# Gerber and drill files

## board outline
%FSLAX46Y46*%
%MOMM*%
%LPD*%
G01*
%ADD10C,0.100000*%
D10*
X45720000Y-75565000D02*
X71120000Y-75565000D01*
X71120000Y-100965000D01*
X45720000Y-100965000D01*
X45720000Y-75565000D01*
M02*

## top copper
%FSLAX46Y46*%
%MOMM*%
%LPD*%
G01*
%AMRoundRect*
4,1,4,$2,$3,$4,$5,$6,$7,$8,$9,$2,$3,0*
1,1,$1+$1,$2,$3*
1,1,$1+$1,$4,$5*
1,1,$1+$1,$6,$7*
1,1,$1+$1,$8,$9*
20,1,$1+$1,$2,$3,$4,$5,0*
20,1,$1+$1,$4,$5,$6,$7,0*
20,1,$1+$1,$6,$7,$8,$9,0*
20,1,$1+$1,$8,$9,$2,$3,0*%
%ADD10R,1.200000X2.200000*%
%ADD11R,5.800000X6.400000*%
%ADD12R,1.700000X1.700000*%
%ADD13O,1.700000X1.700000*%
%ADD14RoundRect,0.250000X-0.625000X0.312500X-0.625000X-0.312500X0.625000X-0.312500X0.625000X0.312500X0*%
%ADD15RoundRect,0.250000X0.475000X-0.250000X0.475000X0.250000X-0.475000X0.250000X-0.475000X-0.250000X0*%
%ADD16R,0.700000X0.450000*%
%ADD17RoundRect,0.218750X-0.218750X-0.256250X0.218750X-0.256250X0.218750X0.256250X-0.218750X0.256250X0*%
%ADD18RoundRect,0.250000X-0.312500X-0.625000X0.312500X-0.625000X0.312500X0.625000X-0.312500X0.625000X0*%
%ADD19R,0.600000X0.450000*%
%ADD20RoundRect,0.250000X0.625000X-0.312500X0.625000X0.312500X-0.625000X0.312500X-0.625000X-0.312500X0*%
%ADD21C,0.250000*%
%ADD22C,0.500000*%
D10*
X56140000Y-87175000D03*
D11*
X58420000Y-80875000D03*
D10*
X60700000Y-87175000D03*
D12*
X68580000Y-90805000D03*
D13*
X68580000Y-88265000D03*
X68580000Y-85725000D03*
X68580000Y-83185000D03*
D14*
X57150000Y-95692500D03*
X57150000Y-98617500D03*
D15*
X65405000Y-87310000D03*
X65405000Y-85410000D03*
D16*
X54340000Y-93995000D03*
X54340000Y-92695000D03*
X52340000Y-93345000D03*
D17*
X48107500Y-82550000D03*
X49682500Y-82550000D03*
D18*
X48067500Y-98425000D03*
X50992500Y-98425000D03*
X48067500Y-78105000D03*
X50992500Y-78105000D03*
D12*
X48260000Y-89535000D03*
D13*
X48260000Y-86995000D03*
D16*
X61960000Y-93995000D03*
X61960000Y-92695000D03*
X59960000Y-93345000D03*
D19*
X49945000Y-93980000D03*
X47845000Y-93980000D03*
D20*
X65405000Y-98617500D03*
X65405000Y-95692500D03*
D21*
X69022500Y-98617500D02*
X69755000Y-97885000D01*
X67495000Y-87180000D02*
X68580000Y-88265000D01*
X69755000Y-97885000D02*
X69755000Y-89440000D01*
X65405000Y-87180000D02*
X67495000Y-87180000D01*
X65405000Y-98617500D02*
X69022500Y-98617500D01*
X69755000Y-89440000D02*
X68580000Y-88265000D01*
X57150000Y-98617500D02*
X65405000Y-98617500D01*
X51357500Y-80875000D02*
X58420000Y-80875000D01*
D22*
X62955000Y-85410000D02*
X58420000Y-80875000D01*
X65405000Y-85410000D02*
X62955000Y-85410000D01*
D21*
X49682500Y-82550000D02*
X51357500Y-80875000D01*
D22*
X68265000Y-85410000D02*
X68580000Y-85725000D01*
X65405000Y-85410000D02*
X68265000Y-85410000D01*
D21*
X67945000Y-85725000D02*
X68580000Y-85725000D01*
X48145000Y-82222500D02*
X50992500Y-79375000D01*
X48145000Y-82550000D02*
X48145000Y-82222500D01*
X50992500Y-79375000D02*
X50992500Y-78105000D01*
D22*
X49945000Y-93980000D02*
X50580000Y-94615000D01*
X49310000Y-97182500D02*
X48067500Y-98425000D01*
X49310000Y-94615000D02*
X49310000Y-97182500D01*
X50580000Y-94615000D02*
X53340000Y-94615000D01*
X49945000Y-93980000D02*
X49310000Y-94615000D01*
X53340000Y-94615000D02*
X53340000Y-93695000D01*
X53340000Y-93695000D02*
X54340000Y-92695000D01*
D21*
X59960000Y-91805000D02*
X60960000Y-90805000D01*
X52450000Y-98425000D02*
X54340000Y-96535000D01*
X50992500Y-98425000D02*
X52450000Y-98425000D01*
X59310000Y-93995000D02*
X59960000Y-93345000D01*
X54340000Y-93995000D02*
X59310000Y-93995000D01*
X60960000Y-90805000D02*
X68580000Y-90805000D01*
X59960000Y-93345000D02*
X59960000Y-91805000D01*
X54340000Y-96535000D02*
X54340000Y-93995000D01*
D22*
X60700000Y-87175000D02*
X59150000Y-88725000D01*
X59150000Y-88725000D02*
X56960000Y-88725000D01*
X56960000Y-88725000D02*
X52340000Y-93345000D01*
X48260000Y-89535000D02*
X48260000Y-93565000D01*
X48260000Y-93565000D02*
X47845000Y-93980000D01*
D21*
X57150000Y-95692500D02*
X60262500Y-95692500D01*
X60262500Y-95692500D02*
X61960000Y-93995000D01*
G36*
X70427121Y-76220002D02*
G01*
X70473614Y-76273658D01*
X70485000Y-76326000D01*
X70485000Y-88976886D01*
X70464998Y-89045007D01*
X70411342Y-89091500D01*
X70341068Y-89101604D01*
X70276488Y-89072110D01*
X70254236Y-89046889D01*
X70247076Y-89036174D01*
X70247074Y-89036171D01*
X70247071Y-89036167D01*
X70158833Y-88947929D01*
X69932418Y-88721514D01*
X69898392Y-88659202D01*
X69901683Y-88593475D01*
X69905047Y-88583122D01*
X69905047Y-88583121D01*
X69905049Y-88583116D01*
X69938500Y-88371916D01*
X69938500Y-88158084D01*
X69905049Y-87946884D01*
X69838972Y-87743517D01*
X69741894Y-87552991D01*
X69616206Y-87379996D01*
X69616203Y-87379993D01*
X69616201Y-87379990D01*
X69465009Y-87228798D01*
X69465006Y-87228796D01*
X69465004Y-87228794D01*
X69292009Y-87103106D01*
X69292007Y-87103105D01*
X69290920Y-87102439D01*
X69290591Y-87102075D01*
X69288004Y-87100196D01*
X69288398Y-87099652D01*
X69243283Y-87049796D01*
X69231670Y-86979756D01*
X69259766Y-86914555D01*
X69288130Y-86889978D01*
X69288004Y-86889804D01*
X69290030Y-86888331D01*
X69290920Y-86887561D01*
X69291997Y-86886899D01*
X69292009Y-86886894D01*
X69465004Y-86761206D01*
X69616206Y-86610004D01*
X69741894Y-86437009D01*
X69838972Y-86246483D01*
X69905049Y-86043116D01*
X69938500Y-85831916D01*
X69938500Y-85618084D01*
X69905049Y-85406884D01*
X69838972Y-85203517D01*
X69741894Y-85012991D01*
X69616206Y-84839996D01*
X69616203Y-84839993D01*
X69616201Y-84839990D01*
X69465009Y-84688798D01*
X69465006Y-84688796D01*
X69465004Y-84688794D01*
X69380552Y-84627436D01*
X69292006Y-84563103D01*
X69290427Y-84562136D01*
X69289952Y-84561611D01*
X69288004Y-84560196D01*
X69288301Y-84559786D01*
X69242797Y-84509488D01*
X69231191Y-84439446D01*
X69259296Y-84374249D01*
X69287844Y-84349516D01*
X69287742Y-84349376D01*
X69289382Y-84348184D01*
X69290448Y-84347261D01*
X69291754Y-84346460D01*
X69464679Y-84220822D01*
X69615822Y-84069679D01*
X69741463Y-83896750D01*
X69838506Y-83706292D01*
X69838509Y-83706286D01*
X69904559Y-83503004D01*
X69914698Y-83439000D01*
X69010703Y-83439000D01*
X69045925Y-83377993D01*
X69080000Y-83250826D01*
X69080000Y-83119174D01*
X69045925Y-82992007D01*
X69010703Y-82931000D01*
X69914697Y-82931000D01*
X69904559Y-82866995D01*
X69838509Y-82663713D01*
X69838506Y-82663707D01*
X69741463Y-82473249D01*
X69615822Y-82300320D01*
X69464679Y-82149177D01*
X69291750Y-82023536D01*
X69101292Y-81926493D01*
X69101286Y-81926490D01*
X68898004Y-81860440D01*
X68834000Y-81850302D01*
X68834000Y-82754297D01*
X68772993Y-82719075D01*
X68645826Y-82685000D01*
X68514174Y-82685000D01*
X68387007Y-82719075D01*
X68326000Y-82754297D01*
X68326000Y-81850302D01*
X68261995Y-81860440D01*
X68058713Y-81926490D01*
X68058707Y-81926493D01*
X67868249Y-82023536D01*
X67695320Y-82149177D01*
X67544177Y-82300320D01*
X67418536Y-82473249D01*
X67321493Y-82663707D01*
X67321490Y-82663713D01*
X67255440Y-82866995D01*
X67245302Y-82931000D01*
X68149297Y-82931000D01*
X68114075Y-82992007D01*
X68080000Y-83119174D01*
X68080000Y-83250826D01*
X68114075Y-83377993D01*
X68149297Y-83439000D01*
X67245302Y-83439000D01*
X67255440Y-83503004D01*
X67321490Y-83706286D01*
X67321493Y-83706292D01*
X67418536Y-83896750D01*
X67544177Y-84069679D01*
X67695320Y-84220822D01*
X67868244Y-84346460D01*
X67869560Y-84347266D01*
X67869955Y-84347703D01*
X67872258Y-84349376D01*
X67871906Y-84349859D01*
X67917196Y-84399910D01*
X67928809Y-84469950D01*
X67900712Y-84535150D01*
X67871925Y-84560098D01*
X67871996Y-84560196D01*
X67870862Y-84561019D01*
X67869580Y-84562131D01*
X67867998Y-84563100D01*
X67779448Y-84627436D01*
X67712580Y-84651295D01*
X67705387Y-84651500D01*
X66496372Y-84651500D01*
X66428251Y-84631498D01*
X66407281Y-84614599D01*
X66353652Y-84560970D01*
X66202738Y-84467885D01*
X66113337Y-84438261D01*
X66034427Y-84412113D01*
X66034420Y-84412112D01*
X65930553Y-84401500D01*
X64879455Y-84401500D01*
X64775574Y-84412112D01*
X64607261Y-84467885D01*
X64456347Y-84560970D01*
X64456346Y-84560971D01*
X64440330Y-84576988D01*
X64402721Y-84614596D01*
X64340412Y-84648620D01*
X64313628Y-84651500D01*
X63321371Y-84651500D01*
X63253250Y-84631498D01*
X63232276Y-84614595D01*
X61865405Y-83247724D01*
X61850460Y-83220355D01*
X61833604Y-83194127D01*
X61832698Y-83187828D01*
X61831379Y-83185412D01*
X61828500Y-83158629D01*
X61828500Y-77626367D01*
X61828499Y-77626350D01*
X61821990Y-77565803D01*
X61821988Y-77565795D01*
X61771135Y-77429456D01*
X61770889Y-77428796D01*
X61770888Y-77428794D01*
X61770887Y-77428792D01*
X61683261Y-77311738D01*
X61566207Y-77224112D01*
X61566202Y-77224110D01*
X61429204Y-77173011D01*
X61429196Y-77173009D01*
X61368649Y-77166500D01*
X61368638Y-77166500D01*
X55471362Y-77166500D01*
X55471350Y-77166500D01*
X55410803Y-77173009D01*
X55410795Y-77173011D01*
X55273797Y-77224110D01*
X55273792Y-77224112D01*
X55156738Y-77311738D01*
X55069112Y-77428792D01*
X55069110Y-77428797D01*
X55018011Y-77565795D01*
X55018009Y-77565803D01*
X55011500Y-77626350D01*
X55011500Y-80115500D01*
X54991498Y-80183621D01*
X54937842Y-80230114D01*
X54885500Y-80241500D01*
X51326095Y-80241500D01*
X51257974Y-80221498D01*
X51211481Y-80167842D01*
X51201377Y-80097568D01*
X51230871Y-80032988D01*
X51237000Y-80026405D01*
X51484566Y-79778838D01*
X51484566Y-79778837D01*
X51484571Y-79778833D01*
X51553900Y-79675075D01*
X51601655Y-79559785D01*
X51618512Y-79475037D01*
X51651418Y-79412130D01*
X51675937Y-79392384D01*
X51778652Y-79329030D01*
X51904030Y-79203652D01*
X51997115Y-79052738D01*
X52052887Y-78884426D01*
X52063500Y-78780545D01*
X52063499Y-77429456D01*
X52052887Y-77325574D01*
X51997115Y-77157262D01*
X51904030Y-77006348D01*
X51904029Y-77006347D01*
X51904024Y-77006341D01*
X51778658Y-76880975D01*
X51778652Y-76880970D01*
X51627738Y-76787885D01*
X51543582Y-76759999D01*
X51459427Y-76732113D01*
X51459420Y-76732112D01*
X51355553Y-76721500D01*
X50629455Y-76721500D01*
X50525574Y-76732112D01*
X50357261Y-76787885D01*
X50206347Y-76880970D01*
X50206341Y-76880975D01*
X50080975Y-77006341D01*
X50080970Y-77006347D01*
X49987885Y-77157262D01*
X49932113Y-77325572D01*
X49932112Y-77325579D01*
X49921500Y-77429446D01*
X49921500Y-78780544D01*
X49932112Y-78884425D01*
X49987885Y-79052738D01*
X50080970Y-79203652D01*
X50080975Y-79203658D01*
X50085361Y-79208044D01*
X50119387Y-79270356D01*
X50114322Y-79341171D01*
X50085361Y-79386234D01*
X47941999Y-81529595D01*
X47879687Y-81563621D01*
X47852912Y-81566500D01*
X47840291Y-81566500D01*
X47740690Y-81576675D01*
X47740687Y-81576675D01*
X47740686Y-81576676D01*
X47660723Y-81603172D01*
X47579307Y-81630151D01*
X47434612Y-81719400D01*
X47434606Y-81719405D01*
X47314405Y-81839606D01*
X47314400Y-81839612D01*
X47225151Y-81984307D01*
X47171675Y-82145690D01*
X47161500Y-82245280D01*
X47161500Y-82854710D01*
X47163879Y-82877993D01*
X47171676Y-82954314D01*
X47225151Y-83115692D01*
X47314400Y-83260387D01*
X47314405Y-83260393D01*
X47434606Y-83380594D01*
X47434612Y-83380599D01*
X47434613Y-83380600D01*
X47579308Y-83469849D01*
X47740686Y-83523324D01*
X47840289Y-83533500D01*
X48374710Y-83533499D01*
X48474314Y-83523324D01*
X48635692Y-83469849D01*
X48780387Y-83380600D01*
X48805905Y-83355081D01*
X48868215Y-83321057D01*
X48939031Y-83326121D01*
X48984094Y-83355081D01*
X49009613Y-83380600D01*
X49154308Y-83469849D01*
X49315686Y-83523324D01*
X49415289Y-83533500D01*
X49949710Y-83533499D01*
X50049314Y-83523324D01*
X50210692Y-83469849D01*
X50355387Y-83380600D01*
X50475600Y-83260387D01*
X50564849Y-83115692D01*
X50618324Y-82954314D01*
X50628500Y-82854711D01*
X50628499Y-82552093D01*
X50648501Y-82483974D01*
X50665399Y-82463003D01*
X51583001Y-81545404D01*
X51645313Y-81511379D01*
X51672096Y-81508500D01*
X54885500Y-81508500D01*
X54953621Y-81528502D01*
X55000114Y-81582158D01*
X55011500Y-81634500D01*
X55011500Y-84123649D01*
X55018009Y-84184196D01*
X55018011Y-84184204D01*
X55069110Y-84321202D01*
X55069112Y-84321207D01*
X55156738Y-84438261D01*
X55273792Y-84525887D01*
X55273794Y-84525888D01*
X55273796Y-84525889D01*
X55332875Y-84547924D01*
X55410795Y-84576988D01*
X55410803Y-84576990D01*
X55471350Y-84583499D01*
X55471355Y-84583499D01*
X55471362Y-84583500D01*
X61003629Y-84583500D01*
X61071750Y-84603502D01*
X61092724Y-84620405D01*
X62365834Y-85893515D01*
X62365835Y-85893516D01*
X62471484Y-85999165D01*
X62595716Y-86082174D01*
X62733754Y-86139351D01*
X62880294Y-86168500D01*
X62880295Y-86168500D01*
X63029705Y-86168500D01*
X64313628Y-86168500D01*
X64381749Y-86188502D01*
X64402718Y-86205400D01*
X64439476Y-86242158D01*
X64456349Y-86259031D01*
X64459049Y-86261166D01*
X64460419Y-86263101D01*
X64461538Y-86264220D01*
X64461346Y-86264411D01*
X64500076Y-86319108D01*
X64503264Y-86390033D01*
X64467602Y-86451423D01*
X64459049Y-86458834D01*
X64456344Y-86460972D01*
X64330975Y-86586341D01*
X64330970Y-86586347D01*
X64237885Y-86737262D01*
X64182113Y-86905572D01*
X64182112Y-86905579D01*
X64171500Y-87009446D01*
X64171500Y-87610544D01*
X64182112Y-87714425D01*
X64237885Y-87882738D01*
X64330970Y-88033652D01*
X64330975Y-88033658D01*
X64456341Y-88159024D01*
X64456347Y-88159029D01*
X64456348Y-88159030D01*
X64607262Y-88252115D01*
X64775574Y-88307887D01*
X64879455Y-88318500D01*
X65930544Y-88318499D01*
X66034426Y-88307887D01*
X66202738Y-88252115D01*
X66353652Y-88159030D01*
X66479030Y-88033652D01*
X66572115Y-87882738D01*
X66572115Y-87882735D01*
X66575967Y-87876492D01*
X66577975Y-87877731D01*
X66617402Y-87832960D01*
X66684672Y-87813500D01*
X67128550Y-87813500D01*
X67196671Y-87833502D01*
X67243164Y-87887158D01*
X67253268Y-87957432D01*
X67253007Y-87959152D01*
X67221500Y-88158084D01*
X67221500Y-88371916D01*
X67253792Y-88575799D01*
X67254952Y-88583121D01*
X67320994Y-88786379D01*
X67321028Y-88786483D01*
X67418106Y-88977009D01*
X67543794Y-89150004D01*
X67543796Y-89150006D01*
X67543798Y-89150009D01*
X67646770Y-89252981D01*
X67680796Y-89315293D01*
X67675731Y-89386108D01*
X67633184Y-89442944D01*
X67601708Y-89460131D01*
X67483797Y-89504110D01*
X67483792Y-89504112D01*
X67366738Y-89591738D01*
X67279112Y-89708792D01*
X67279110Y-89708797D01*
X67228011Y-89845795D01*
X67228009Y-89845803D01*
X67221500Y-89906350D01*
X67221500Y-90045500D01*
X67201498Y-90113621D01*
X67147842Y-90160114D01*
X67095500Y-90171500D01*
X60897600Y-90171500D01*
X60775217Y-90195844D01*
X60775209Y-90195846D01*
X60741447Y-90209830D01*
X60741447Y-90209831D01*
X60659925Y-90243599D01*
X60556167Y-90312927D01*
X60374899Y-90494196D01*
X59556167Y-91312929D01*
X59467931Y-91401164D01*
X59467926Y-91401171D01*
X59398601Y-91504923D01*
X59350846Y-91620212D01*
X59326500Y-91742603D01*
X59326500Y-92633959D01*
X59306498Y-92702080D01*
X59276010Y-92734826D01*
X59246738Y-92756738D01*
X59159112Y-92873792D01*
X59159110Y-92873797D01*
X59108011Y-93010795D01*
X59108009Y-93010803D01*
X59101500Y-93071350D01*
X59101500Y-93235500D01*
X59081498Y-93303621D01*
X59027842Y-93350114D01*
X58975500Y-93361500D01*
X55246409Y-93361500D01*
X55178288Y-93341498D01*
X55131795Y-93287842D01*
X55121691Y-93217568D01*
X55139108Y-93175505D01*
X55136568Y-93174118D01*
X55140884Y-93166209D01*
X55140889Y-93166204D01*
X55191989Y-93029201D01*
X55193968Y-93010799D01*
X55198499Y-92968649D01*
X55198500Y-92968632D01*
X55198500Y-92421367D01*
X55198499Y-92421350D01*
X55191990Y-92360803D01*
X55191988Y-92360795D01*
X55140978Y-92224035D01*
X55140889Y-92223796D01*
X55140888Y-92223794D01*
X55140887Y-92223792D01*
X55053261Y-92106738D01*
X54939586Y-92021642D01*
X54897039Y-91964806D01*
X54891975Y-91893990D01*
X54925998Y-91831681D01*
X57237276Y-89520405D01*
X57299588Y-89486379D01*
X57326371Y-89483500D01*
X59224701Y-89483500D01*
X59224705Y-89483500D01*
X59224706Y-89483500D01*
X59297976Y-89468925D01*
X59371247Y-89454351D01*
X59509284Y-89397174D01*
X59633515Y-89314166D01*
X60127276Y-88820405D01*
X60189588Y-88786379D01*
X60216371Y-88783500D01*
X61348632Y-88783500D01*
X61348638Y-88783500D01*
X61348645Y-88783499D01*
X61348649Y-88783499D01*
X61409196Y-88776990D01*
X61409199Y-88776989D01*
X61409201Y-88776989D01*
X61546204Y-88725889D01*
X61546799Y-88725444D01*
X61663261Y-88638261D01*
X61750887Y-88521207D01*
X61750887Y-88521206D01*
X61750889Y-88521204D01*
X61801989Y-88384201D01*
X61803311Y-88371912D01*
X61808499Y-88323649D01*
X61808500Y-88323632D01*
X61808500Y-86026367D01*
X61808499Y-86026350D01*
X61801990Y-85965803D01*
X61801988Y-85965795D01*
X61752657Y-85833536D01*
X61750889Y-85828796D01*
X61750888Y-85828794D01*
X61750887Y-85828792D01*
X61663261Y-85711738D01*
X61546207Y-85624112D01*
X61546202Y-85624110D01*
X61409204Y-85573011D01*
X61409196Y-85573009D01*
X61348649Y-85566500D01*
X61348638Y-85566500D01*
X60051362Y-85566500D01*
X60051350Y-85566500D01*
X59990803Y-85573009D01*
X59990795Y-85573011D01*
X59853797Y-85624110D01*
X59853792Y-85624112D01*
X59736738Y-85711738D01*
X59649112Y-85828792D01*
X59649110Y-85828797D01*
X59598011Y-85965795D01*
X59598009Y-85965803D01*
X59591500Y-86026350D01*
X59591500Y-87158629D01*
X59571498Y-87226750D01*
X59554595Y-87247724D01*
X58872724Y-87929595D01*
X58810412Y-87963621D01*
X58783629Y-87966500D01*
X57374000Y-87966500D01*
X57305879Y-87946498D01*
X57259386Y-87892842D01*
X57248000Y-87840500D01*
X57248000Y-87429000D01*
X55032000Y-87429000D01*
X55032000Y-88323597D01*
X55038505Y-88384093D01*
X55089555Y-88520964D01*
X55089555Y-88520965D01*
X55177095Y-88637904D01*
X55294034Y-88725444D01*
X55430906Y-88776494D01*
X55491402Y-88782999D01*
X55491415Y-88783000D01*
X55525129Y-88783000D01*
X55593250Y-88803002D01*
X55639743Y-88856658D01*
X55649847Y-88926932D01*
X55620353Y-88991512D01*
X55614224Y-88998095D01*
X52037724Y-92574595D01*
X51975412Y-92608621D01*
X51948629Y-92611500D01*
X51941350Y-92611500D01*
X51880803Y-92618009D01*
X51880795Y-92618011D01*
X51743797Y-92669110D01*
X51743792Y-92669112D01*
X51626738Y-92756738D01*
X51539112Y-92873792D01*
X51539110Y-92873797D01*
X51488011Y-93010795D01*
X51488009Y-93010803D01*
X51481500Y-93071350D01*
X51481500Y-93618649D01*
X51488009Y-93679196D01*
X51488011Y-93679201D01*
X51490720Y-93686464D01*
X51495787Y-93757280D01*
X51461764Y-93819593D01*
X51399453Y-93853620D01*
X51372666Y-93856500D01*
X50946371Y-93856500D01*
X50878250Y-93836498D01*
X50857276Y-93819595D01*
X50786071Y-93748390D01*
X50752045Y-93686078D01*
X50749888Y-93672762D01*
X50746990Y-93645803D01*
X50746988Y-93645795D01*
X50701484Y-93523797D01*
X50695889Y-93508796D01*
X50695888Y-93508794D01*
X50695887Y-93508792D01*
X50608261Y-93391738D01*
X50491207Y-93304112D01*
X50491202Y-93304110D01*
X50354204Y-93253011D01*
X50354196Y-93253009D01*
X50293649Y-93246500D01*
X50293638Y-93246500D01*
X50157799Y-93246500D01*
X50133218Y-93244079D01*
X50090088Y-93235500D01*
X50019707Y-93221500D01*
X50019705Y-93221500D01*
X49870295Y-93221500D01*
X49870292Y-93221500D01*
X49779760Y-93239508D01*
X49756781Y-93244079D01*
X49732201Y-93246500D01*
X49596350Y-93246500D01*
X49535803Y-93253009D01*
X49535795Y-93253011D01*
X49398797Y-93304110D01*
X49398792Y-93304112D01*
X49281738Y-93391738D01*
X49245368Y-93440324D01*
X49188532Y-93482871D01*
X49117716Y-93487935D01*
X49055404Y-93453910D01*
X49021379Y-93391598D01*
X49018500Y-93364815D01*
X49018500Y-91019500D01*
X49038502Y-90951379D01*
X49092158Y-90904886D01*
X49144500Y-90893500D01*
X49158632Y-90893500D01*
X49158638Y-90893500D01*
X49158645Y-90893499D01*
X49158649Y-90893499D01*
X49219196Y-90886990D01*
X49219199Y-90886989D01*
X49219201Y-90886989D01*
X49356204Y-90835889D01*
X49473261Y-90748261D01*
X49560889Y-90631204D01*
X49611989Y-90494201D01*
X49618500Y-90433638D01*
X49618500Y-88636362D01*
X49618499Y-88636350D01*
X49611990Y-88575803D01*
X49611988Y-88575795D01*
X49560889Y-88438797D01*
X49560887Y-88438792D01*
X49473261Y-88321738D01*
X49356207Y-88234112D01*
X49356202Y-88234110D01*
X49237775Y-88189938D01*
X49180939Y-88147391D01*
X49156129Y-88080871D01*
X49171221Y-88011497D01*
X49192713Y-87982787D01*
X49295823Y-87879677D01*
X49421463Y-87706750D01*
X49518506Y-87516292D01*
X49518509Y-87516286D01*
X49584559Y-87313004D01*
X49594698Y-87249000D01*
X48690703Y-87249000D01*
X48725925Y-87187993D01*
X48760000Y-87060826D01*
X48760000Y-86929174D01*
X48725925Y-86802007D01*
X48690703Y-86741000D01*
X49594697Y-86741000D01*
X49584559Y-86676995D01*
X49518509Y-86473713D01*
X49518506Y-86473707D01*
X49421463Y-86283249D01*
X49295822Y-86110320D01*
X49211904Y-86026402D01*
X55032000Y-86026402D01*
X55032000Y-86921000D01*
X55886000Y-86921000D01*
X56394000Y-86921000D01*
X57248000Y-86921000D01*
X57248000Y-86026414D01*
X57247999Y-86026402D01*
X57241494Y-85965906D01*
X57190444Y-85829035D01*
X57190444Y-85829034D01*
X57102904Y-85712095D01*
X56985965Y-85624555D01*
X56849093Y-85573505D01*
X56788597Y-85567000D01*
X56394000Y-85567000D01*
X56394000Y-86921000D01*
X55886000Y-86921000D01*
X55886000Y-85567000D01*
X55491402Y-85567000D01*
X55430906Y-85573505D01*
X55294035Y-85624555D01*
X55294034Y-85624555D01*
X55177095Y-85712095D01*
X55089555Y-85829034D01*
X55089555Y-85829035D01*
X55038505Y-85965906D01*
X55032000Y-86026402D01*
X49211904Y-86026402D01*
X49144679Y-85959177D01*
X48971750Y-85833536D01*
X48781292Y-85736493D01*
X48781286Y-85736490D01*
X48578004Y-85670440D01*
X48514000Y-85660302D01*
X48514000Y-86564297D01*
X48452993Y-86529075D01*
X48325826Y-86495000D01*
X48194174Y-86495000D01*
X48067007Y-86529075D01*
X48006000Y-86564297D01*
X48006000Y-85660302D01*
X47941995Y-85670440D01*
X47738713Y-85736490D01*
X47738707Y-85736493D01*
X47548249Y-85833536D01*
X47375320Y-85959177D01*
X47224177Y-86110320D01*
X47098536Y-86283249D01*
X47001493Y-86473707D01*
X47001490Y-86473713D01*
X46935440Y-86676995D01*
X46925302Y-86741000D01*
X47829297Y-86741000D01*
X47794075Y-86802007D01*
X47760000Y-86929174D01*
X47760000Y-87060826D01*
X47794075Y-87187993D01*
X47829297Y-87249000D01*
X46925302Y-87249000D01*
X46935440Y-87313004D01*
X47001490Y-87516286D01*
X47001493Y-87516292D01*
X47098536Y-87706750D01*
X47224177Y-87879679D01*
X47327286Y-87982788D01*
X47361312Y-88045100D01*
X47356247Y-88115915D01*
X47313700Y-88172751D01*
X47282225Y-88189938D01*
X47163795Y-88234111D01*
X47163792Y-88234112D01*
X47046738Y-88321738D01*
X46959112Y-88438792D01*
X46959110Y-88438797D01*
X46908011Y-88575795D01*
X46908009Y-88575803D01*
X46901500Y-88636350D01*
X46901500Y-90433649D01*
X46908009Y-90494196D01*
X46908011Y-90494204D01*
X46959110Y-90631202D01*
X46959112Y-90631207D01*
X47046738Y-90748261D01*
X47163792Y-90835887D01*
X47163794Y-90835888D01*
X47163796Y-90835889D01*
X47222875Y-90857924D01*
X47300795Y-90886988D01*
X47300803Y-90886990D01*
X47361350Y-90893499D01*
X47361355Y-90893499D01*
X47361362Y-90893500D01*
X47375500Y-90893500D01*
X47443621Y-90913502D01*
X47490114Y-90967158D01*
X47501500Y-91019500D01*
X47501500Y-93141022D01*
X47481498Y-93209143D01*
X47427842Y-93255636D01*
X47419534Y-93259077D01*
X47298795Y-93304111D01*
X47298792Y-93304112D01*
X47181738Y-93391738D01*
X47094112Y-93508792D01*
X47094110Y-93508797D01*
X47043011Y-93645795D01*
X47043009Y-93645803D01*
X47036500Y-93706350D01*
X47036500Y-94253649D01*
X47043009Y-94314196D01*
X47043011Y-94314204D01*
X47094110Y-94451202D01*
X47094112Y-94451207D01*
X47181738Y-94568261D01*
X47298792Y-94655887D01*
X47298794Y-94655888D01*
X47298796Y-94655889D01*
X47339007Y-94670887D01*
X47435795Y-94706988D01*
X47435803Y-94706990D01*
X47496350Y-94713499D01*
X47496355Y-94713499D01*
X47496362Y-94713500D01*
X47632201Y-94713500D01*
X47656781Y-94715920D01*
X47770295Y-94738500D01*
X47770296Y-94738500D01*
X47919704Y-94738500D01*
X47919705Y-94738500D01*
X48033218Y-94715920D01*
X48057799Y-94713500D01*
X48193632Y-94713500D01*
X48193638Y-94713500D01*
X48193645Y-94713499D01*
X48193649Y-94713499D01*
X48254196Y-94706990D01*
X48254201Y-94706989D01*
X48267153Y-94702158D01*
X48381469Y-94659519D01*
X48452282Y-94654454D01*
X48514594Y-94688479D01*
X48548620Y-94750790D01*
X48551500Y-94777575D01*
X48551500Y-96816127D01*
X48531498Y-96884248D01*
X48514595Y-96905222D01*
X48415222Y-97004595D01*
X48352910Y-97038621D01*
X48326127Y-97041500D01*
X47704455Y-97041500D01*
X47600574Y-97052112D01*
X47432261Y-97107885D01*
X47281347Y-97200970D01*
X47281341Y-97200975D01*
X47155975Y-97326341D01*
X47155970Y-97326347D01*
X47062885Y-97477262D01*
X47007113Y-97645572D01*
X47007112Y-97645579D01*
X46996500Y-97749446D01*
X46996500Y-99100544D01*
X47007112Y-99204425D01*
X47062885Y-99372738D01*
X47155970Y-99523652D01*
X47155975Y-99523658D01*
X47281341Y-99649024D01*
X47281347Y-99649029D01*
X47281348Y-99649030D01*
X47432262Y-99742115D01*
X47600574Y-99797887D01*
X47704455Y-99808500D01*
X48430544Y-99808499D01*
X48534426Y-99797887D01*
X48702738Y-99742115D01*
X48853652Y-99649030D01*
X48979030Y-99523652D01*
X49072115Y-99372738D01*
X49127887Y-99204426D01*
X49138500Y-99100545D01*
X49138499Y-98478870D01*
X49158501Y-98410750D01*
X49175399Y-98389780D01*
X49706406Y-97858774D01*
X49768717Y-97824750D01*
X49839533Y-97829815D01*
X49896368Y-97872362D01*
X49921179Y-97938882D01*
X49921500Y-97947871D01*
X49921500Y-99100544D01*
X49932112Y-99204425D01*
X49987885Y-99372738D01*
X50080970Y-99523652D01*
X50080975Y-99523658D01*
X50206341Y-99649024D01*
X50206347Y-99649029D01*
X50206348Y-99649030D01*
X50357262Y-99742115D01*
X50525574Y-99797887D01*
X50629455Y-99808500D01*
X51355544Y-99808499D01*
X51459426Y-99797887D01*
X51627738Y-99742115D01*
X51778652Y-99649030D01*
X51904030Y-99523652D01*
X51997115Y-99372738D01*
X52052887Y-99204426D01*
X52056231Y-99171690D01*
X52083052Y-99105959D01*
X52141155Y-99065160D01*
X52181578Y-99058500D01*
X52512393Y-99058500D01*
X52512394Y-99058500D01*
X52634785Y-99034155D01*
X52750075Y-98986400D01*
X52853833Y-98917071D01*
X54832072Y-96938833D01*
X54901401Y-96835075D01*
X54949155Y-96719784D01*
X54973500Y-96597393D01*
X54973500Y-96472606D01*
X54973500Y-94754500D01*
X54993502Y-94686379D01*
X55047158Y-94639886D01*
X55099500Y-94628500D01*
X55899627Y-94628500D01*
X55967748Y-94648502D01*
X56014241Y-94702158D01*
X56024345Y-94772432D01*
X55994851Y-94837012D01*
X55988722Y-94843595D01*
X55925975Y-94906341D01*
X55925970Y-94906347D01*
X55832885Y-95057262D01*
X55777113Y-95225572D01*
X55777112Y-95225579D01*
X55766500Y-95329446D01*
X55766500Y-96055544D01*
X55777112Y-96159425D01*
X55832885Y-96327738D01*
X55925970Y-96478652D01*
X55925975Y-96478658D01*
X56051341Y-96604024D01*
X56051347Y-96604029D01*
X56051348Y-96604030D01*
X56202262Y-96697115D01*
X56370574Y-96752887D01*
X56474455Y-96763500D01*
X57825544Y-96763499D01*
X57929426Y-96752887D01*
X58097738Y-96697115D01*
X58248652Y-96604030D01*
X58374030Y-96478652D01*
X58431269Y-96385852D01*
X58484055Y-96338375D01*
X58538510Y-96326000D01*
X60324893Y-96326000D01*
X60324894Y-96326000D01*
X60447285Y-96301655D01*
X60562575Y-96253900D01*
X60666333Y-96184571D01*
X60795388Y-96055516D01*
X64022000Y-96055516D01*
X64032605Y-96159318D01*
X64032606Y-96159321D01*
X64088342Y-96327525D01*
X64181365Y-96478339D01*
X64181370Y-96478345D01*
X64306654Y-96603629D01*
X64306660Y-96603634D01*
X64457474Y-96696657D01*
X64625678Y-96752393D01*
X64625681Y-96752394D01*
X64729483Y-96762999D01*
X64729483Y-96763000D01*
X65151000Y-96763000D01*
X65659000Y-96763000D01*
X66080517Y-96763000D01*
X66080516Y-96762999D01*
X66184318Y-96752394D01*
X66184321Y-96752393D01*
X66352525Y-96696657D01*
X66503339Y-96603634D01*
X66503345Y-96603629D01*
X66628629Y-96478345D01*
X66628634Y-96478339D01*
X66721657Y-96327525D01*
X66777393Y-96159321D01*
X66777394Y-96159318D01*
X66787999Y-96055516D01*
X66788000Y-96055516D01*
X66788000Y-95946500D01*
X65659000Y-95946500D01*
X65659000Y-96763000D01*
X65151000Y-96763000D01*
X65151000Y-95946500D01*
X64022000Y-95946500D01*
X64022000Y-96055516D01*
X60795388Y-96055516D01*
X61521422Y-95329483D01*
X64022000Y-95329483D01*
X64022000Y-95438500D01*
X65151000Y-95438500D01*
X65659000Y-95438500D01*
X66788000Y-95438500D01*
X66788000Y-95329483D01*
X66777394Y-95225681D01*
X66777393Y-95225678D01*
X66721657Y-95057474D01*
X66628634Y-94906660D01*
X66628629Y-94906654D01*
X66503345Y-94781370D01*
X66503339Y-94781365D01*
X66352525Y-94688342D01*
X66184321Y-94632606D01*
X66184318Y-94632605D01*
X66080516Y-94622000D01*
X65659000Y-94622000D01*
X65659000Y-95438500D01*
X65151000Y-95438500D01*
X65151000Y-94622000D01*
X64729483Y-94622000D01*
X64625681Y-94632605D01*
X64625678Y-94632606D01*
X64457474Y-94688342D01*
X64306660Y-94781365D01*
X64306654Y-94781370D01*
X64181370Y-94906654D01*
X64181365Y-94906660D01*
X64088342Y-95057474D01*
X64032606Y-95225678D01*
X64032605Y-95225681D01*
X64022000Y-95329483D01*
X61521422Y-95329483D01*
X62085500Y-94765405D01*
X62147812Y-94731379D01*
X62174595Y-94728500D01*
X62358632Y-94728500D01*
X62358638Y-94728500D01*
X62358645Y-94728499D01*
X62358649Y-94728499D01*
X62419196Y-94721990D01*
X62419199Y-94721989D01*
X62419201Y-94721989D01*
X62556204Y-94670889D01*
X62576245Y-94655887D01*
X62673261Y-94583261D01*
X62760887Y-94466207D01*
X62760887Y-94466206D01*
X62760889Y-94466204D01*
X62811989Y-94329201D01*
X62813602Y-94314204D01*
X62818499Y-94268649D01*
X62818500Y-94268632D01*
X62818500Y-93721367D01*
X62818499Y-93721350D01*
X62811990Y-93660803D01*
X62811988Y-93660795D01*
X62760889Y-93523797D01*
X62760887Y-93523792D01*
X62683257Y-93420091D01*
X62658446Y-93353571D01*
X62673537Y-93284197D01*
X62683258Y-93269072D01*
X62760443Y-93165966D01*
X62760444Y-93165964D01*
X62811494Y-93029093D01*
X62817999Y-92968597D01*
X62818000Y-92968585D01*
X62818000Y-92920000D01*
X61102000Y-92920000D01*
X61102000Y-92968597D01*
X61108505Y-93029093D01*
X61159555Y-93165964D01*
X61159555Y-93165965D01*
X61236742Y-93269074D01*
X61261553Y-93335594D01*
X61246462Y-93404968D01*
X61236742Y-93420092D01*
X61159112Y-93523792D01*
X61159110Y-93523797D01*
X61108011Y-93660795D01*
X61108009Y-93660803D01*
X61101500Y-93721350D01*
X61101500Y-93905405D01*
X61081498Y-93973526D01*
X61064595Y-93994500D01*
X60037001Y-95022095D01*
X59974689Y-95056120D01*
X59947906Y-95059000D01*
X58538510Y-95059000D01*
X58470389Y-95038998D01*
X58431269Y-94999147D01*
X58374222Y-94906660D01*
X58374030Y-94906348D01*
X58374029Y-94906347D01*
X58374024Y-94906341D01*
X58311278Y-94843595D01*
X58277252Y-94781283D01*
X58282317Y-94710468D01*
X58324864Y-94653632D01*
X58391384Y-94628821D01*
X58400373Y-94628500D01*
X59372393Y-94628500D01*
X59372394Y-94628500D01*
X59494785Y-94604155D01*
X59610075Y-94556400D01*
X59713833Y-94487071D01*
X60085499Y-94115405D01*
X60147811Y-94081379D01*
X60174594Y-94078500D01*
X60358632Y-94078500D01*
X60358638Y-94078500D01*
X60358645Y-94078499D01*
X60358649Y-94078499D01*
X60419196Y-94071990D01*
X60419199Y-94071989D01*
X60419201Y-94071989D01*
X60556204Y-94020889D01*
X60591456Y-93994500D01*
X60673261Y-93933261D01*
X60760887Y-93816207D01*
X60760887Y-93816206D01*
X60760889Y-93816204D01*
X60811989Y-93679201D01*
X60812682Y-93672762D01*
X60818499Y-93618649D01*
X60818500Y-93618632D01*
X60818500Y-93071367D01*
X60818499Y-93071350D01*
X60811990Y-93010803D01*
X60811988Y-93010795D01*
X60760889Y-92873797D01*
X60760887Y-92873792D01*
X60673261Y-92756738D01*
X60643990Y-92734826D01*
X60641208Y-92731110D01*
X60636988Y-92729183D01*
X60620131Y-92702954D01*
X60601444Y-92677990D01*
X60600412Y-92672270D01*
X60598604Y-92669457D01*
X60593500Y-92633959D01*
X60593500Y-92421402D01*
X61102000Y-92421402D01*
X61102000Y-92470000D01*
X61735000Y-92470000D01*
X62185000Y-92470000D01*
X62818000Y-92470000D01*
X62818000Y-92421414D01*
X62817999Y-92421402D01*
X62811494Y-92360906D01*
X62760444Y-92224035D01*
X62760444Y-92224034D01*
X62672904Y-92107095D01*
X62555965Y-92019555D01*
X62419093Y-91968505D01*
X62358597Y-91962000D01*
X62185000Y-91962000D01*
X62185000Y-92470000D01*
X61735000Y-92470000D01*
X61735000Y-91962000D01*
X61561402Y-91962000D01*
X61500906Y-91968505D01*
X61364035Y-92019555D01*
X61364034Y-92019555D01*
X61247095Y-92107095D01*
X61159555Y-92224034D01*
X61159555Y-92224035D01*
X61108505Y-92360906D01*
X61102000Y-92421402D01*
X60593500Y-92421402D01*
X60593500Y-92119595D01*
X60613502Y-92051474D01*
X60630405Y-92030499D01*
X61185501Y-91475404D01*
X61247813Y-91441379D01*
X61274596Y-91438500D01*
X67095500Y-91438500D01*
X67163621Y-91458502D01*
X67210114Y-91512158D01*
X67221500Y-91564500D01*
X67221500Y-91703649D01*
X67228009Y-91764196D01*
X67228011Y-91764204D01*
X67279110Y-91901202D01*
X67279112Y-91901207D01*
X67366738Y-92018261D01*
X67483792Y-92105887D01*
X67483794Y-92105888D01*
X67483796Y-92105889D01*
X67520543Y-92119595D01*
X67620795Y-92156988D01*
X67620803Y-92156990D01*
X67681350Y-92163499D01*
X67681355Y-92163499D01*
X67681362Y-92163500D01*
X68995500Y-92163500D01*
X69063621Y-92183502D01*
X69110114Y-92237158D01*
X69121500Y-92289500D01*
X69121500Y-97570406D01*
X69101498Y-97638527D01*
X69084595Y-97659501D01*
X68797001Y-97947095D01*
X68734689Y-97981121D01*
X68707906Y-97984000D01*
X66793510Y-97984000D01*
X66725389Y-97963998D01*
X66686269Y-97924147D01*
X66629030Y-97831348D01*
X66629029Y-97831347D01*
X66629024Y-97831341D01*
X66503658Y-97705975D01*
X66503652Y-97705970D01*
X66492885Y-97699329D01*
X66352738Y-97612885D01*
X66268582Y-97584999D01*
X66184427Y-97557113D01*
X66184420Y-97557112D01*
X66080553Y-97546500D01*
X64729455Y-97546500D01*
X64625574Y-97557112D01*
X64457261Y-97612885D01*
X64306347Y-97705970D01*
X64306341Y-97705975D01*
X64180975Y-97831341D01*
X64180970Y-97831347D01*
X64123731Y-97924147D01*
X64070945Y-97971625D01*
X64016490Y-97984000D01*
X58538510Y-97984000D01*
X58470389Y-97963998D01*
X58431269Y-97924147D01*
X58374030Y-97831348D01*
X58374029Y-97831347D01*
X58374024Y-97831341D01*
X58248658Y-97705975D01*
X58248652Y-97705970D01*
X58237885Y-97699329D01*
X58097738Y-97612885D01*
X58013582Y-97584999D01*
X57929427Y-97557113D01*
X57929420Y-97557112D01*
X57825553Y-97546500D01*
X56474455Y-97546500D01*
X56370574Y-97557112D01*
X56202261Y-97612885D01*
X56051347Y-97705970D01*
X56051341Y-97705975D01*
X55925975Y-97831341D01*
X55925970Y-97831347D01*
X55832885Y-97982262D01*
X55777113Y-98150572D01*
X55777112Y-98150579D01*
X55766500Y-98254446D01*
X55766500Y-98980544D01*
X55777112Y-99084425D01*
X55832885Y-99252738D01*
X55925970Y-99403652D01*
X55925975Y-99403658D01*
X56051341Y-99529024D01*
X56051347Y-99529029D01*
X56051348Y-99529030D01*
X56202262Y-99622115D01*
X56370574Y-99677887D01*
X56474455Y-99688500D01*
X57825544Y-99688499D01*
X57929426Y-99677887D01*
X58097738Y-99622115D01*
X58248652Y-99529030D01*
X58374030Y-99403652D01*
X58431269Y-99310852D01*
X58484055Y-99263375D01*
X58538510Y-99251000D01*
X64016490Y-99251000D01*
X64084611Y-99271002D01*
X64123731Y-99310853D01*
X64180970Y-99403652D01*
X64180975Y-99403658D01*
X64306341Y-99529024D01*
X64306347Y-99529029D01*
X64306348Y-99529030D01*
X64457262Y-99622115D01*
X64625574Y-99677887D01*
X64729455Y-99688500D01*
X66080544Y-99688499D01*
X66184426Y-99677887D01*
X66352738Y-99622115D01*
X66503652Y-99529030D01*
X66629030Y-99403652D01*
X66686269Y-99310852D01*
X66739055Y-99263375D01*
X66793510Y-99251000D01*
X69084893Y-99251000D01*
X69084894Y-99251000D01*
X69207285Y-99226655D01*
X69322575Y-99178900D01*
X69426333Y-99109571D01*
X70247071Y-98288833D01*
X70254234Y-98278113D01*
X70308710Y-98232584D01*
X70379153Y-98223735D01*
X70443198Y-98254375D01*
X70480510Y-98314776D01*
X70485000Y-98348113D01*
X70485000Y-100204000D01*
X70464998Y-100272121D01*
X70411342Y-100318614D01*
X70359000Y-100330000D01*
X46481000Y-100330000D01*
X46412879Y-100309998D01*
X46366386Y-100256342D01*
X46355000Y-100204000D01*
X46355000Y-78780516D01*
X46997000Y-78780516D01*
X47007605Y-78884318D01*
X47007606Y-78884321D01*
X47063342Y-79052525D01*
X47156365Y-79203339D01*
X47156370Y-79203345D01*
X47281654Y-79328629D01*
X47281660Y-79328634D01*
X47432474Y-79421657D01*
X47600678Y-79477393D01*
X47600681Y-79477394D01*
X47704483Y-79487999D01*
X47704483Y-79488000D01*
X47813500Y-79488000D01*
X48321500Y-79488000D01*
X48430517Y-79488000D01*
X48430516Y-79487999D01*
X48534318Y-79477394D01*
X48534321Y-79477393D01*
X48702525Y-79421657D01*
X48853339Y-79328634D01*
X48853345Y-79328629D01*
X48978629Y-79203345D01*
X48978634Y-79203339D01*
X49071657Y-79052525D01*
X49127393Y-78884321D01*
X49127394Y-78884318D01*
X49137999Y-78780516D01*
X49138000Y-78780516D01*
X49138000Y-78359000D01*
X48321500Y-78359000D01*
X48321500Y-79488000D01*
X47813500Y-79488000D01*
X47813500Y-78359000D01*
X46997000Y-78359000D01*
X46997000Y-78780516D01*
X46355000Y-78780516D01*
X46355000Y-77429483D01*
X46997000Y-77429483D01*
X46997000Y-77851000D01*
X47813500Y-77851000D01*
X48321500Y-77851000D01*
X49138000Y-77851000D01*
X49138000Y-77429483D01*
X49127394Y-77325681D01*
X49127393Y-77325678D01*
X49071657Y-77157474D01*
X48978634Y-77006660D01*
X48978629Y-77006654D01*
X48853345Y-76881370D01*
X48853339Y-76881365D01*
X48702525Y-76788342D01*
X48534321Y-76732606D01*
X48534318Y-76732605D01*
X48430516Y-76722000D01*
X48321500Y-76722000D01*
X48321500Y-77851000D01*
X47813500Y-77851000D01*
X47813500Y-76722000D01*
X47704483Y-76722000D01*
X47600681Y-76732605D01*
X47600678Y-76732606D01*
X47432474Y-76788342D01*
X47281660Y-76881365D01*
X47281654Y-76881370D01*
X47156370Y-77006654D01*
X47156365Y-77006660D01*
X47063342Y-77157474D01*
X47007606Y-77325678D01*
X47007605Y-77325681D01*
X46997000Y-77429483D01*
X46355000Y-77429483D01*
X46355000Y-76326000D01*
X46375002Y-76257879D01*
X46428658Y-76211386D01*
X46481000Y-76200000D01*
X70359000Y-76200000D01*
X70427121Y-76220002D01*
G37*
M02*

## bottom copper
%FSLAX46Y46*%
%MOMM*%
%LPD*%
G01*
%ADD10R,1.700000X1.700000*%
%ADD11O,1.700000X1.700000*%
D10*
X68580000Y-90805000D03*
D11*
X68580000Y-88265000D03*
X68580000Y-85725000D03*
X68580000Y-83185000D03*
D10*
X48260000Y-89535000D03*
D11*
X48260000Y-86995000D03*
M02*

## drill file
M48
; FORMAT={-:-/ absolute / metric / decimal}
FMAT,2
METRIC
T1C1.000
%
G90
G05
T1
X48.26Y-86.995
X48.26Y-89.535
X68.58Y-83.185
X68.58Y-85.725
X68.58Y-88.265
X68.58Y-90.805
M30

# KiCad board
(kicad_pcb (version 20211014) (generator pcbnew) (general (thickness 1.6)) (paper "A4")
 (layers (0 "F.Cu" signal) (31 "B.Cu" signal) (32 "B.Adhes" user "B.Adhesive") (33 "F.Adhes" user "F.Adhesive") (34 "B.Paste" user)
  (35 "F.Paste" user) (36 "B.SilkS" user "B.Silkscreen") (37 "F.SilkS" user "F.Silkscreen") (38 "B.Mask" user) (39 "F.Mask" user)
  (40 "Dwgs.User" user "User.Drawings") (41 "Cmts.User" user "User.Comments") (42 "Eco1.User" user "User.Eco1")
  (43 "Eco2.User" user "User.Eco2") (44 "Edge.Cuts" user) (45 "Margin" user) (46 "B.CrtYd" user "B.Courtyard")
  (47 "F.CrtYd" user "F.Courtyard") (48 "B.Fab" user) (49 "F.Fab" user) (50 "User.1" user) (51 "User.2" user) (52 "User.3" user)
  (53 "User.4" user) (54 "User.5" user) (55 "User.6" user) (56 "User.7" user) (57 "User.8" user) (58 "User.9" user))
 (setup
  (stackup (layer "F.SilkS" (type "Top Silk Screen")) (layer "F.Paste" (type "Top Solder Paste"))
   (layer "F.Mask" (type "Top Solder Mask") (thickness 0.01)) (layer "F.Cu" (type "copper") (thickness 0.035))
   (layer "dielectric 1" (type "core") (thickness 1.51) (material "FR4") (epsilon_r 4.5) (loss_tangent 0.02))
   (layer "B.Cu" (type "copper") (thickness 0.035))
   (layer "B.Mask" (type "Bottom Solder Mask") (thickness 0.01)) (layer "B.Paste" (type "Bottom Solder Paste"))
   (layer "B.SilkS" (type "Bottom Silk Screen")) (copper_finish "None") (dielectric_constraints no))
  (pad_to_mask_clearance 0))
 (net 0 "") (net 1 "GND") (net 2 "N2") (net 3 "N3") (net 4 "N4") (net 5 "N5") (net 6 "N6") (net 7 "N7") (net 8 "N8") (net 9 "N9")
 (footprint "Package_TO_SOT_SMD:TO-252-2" (layer "F.Cu") (at 58.42 82.975 90)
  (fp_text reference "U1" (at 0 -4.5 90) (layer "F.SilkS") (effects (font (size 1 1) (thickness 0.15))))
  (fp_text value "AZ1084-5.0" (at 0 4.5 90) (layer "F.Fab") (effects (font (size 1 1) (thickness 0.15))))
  (pad "" smd rect (at 0.425 -1.525 90) (size 3.05 2.75) (layers "F.Paste"))
  (pad "" smd rect (at 3.775 -1.525 90) (size 3.05 2.75) (layers "F.Paste"))
  (pad "" smd rect (at 3.775 1.525 90) (size 3.05 2.75) (layers "F.Paste"))
  (pad "" smd rect (at 0.425 1.525 90) (size 3.05 2.75) (layers "F.Paste"))
  (pad "1" smd rect (at -4.2 -2.28 90) (size 2.2 1.2) (layers "F.Cu" "F.Paste" "F.Mask") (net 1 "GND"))
  (pad "2" smd rect (at 2.1 0 90) (size 6.4 5.8) (layers "F.Cu" "F.Mask") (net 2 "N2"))
  (pad "3" smd rect (at -4.2 2.28 90) (size 2.2 1.2) (layers "F.Cu" "F.Paste" "F.Mask") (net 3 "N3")))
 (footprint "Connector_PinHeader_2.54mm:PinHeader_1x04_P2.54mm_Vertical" (layer "F.Cu") (at 68.58 90.805 180)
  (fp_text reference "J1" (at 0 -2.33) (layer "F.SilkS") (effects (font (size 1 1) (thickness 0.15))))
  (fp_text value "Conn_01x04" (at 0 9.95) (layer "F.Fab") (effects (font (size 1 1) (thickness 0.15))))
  (pad "1" thru_hole rect (at 0 0 180) (size 1.7 1.7) (drill 1) (layers *.Cu *.Mask) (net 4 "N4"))
  (pad "2" thru_hole oval (at 0 2.54 180) (size 1.7 1.7) (drill 1) (layers *.Cu *.Mask) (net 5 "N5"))
  (pad "3" thru_hole oval (at 0 5.08 180) (size 1.7 1.7) (drill 1) (layers *.Cu *.Mask) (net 2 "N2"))
  (pad "4" thru_hole oval (at 0 7.62 180) (size 1.7 1.7) (drill 1) (layers *.Cu *.Mask) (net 1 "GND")))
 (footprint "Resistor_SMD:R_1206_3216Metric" (layer "F.Cu") (at 57.15 97.155 -90)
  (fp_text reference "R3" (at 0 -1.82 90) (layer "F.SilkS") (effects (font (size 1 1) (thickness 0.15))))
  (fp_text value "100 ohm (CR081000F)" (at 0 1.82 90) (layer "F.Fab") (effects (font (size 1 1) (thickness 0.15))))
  (pad "1" smd roundrect (at -1.4625 0 270) (size 1.125 1.75) (layers "F.Cu" "F.Paste" "F.Mask") (roundrect_rratio 0.2222222222)
   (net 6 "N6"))
  (pad "2" smd roundrect (at 1.4625 0 270) (size 1.125 1.75) (layers "F.Cu" "F.Paste" "F.Mask") (roundrect_rratio 0.2222222222) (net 5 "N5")))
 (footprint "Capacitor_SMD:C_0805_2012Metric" (layer "F.Cu") (at 65.405 86.36 90)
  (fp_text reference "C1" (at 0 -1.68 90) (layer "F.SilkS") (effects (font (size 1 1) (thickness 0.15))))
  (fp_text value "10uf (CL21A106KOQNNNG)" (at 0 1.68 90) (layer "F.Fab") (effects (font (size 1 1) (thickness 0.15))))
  (pad "1" smd roundrect (at -0.95 0 90) (size 1 1.45) (layers "F.Cu" "F.Paste" "F.Mask") (roundrect_rratio 0.25) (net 5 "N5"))
  (pad "2" smd roundrect (at 0.95 0 90) (size 1 1.45) (layers "F.Cu" "F.Paste" "F.Mask") (roundrect_rratio 0.25) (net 2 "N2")))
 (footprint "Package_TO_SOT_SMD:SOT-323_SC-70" (layer "F.Cu") (at 53.34 93.345 180)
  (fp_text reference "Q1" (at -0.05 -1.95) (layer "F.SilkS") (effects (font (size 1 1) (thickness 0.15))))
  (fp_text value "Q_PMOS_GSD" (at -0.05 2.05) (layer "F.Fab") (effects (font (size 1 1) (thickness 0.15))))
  (pad "1" smd rect (at -1 -0.65 90) (size 0.45 0.7) (layers "F.Cu" "F.Paste" "F.Mask") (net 4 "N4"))
  (pad "2" smd rect (at -1 0.65 90) (size 0.45 0.7) (layers "F.Cu" "F.Paste" "F.Mask") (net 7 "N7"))
  (pad "3" smd rect (at 1 0 90) (size 0.45 0.7) (layers "F.Cu" "F.Paste" "F.Mask") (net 3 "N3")))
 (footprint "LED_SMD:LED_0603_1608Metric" (layer "F.Cu") (at 48.895 82.55)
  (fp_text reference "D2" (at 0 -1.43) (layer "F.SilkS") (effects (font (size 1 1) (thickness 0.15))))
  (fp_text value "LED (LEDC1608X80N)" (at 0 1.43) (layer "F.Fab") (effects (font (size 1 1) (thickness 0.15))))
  (pad "1" smd roundrect (at -0.7875 0) (size 0.875 0.95) (layers "F.Cu" "F.Paste" "F.Mask") (roundrect_rratio 0.25) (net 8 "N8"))
  (pad "2" smd roundrect (at 0.7875 0) (size 0.875 0.95) (layers "F.Cu" "F.Paste" "F.Mask") (roundrect_rratio 0.25) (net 2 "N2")))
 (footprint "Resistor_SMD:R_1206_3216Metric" (layer "F.Cu") (at 49.53 98.425)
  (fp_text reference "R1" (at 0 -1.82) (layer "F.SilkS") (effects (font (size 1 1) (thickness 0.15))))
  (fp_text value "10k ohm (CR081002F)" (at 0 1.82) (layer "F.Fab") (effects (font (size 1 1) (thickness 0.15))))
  (pad "1" smd roundrect (at -1.4625 0) (size 1.125 1.75) (layers "F.Cu" "F.Paste" "F.Mask") (roundrect_rratio 0.2222222222) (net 7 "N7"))
  (pad "2" smd roundrect (at 1.4625 0) (size 1.125 1.75) (layers "F.Cu" "F.Paste" "F.Mask") (roundrect_rratio 0.2222222222) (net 4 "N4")))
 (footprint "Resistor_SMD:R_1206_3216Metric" (layer "F.Cu") (at 49.53 78.105)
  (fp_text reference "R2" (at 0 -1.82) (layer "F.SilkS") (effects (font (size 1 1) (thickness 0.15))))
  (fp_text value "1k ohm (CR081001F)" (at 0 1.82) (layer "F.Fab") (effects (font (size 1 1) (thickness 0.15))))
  (pad "1" smd roundrect (at -1.4625 0) (size 1.125 1.75) (layers "F.Cu" "F.Paste" "F.Mask") (roundrect_rratio 0.2222222222) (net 1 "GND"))
  (pad "2" smd roundrect (at 1.4625 0) (size 1.125 1.75) (layers "F.Cu" "F.Paste" "F.Mask") (roundrect_rratio 0.2222222222) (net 8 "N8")))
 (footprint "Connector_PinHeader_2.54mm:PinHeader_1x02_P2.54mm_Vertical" (layer "F.Cu") (at 48.26 89.535 180)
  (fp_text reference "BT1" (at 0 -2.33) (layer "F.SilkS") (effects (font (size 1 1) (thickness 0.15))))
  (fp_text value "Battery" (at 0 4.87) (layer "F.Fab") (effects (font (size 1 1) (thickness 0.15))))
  (pad "1" thru_hole rect (at 0 0 180) (size 1.7 1.7) (drill 1) (layers *.Cu *.Mask) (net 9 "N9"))
  (pad "2" thru_hole oval (at 0 2.54 180) (size 1.7 1.7) (drill 1) (layers *.Cu *.Mask) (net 1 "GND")))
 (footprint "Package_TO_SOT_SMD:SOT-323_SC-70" (layer "F.Cu") (at 60.96 93.345 180)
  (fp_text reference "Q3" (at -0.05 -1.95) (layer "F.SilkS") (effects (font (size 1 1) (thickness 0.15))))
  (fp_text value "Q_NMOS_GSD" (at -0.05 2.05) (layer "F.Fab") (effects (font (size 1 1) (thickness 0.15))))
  (pad "1" smd rect (at -1 -0.65 90) (size 0.45 0.7) (layers "F.Cu" "F.Paste" "F.Mask") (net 6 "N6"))
  (pad "2" smd rect (at -1 0.65 90) (size 0.45 0.7) (layers "F.Cu" "F.Paste" "F.Mask") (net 1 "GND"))
  (pad "3" smd rect (at 1 0 90) (size 0.45 0.7) (layers "F.Cu" "F.Paste" "F.Mask") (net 4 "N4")))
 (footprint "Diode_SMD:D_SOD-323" (layer "F.Cu") (at 48.895 93.98 180)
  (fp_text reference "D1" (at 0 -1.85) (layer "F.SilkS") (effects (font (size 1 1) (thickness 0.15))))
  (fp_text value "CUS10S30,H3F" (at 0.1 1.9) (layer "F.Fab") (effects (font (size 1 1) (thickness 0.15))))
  (pad "1" smd rect (at -1.05 0 180) (size 0.6 0.45) (layers "F.Cu" "F.Paste" "F.Mask") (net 7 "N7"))
  (pad "2" smd rect (at 1.05 0 180) (size 0.6 0.45) (layers "F.Cu" "F.Paste" "F.Mask") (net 9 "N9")))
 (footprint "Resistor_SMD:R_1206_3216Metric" (layer "F.Cu") (at 65.405 97.155 90)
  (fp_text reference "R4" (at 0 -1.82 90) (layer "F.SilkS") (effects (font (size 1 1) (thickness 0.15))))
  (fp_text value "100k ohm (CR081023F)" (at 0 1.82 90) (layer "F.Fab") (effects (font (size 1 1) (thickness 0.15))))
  (pad "1" smd roundrect (at -1.4625 0 90) (size 1.125 1.75) (layers "F.Cu" "F.Paste" "F.Mask") (roundrect_rratio 0.2222222222) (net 5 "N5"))
  (pad "2" smd roundrect (at 1.4625 0 90) (size 1.125 1.75) (layers "F.Cu" "F.Paste" "F.Mask") (roundrect_rratio 0.2222222222) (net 1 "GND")))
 (gr_rect (start 45.72 100.965) (end 71.12 75.565) (layer "Edge.Cuts") (width 0.1) (fill none))
 (segment (start 69.0225 98.6175) (end 69.755 97.885) (width 0.25) (layer "F.Cu") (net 5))
 (segment (start 67.495 87.18) (end 68.58 88.265) (width 0.25) (layer "F.Cu") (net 5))
 (segment (start 69.755 97.885) (end 69.755 89.44) (width 0.25) (layer "F.Cu") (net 5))
 (segment (start 65.405 87.18) (end 67.495 87.18) (width 0.25) (layer "F.Cu") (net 5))
 (segment (start 65.405 98.6175) (end 69.0225 98.6175) (width 0.25) (layer "F.Cu") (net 5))
 (segment (start 69.755 89.44) (end 68.58 88.265) (width 0.25) (layer "F.Cu") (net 5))
 (segment (start 57.15 98.6175) (end 65.405 98.6175) (width 0.25) (layer "F.Cu") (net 5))
 (segment (start 51.3575 80.875) (end 58.42 80.875) (width 0.25) (layer "F.Cu") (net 2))
 (segment (start 62.955 85.41) (end 58.42 80.875) (width 0.5) (layer "F.Cu") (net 2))
 (segment (start 65.405 85.41) (end 62.955 85.41) (width 0.5) (layer "F.Cu") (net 2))
 (segment (start 49.6825 82.55) (end 51.3575 80.875) (width 0.25) (layer "F.Cu") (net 2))
 (segment (start 68.265 85.41) (end 68.58 85.725) (width 0.5) (layer "F.Cu") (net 2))
 (segment (start 65.405 85.41) (end 68.265 85.41) (width 0.5) (layer "F.Cu") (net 2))
 (segment (start 67.945 85.725) (end 68.58 85.725) (width 0.25) (layer "F.Cu") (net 2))
 (segment (start 48.145 82.2225) (end 50.9925 79.375) (width 0.25) (layer "F.Cu") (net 8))
 (segment (start 48.145 82.55) (end 48.145 82.2225) (width 0.25) (layer "F.Cu") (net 8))
 (segment (start 50.9925 79.375) (end 50.9925 78.105) (width 0.25) (layer "F.Cu") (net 8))
 (segment (start 49.945 93.98) (end 50.58 94.615) (width 0.5) (layer "F.Cu") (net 7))
 (segment (start 49.31 97.1825) (end 48.0675 98.425) (width 0.5) (layer "F.Cu") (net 7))
 (segment (start 49.31 94.615) (end 49.31 97.1825) (width 0.5) (layer "F.Cu") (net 7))
 (segment (start 50.58 94.615) (end 53.34 94.615) (width 0.5) (layer "F.Cu") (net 7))
 (segment (start 49.945 93.98) (end 49.31 94.615) (width 0.5) (layer "F.Cu") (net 7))
 (segment (start 53.34 94.615) (end 53.34 93.695) (width 0.5) (layer "F.Cu") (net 7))
 (segment (start 53.34 93.695) (end 54.34 92.695) (width 0.5) (layer "F.Cu") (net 7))
 (segment (start 59.96 91.805) (end 60.96 90.805) (width 0.25) (layer "F.Cu") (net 4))
 (segment (start 52.45 98.425) (end 54.34 96.535) (width 0.25) (layer "F.Cu") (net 4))
 (segment (start 50.9925 98.425) (end 52.45 98.425) (width 0.25) (layer "F.Cu") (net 4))
 (segment (start 59.31 93.995) (end 59.96 93.345) (width 0.25) (layer "F.Cu") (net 4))
 (segment (start 54.34 93.995) (end 59.31 93.995) (width 0.25) (layer "F.Cu") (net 4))
 (segment (start 60.96 90.805) (end 68.58 90.805) (width 0.25) (layer "F.Cu") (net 4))
 (segment (start 59.96 93.345) (end 59.96 91.805) (width 0.25) (layer "F.Cu") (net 4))
 (segment (start 54.34 96.535) (end 54.34 93.995) (width 0.25) (layer "F.Cu") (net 4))
 (segment (start 60.7 87.175) (end 59.15 88.725) (width 0.5) (layer "F.Cu") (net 3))
 (segment (start 59.15 88.725) (end 56.96 88.725) (width 0.5) (layer "F.Cu") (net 3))
 (segment (start 56.96 88.725) (end 52.34 93.345) (width 0.5) (layer "F.Cu") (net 3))
 (segment (start 48.26 89.535) (end 48.26 93.565) (width 0.5) (layer "F.Cu") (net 9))
 (segment (start 48.26 93.565) (end 47.845 93.98) (width 0.5) (layer "F.Cu") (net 9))
 (segment (start 57.15 95.6925) (end 60.2625 95.6925) (width 0.25) (layer "F.Cu") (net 6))
 (segment (start 60.2625 95.6925) (end 61.96 93.995) (width 0.25) (layer "F.Cu") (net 6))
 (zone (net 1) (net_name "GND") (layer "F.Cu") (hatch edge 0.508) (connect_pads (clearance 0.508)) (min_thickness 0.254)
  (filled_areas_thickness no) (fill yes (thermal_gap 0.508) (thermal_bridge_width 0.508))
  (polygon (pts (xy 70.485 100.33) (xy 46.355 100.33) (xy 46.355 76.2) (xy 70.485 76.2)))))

